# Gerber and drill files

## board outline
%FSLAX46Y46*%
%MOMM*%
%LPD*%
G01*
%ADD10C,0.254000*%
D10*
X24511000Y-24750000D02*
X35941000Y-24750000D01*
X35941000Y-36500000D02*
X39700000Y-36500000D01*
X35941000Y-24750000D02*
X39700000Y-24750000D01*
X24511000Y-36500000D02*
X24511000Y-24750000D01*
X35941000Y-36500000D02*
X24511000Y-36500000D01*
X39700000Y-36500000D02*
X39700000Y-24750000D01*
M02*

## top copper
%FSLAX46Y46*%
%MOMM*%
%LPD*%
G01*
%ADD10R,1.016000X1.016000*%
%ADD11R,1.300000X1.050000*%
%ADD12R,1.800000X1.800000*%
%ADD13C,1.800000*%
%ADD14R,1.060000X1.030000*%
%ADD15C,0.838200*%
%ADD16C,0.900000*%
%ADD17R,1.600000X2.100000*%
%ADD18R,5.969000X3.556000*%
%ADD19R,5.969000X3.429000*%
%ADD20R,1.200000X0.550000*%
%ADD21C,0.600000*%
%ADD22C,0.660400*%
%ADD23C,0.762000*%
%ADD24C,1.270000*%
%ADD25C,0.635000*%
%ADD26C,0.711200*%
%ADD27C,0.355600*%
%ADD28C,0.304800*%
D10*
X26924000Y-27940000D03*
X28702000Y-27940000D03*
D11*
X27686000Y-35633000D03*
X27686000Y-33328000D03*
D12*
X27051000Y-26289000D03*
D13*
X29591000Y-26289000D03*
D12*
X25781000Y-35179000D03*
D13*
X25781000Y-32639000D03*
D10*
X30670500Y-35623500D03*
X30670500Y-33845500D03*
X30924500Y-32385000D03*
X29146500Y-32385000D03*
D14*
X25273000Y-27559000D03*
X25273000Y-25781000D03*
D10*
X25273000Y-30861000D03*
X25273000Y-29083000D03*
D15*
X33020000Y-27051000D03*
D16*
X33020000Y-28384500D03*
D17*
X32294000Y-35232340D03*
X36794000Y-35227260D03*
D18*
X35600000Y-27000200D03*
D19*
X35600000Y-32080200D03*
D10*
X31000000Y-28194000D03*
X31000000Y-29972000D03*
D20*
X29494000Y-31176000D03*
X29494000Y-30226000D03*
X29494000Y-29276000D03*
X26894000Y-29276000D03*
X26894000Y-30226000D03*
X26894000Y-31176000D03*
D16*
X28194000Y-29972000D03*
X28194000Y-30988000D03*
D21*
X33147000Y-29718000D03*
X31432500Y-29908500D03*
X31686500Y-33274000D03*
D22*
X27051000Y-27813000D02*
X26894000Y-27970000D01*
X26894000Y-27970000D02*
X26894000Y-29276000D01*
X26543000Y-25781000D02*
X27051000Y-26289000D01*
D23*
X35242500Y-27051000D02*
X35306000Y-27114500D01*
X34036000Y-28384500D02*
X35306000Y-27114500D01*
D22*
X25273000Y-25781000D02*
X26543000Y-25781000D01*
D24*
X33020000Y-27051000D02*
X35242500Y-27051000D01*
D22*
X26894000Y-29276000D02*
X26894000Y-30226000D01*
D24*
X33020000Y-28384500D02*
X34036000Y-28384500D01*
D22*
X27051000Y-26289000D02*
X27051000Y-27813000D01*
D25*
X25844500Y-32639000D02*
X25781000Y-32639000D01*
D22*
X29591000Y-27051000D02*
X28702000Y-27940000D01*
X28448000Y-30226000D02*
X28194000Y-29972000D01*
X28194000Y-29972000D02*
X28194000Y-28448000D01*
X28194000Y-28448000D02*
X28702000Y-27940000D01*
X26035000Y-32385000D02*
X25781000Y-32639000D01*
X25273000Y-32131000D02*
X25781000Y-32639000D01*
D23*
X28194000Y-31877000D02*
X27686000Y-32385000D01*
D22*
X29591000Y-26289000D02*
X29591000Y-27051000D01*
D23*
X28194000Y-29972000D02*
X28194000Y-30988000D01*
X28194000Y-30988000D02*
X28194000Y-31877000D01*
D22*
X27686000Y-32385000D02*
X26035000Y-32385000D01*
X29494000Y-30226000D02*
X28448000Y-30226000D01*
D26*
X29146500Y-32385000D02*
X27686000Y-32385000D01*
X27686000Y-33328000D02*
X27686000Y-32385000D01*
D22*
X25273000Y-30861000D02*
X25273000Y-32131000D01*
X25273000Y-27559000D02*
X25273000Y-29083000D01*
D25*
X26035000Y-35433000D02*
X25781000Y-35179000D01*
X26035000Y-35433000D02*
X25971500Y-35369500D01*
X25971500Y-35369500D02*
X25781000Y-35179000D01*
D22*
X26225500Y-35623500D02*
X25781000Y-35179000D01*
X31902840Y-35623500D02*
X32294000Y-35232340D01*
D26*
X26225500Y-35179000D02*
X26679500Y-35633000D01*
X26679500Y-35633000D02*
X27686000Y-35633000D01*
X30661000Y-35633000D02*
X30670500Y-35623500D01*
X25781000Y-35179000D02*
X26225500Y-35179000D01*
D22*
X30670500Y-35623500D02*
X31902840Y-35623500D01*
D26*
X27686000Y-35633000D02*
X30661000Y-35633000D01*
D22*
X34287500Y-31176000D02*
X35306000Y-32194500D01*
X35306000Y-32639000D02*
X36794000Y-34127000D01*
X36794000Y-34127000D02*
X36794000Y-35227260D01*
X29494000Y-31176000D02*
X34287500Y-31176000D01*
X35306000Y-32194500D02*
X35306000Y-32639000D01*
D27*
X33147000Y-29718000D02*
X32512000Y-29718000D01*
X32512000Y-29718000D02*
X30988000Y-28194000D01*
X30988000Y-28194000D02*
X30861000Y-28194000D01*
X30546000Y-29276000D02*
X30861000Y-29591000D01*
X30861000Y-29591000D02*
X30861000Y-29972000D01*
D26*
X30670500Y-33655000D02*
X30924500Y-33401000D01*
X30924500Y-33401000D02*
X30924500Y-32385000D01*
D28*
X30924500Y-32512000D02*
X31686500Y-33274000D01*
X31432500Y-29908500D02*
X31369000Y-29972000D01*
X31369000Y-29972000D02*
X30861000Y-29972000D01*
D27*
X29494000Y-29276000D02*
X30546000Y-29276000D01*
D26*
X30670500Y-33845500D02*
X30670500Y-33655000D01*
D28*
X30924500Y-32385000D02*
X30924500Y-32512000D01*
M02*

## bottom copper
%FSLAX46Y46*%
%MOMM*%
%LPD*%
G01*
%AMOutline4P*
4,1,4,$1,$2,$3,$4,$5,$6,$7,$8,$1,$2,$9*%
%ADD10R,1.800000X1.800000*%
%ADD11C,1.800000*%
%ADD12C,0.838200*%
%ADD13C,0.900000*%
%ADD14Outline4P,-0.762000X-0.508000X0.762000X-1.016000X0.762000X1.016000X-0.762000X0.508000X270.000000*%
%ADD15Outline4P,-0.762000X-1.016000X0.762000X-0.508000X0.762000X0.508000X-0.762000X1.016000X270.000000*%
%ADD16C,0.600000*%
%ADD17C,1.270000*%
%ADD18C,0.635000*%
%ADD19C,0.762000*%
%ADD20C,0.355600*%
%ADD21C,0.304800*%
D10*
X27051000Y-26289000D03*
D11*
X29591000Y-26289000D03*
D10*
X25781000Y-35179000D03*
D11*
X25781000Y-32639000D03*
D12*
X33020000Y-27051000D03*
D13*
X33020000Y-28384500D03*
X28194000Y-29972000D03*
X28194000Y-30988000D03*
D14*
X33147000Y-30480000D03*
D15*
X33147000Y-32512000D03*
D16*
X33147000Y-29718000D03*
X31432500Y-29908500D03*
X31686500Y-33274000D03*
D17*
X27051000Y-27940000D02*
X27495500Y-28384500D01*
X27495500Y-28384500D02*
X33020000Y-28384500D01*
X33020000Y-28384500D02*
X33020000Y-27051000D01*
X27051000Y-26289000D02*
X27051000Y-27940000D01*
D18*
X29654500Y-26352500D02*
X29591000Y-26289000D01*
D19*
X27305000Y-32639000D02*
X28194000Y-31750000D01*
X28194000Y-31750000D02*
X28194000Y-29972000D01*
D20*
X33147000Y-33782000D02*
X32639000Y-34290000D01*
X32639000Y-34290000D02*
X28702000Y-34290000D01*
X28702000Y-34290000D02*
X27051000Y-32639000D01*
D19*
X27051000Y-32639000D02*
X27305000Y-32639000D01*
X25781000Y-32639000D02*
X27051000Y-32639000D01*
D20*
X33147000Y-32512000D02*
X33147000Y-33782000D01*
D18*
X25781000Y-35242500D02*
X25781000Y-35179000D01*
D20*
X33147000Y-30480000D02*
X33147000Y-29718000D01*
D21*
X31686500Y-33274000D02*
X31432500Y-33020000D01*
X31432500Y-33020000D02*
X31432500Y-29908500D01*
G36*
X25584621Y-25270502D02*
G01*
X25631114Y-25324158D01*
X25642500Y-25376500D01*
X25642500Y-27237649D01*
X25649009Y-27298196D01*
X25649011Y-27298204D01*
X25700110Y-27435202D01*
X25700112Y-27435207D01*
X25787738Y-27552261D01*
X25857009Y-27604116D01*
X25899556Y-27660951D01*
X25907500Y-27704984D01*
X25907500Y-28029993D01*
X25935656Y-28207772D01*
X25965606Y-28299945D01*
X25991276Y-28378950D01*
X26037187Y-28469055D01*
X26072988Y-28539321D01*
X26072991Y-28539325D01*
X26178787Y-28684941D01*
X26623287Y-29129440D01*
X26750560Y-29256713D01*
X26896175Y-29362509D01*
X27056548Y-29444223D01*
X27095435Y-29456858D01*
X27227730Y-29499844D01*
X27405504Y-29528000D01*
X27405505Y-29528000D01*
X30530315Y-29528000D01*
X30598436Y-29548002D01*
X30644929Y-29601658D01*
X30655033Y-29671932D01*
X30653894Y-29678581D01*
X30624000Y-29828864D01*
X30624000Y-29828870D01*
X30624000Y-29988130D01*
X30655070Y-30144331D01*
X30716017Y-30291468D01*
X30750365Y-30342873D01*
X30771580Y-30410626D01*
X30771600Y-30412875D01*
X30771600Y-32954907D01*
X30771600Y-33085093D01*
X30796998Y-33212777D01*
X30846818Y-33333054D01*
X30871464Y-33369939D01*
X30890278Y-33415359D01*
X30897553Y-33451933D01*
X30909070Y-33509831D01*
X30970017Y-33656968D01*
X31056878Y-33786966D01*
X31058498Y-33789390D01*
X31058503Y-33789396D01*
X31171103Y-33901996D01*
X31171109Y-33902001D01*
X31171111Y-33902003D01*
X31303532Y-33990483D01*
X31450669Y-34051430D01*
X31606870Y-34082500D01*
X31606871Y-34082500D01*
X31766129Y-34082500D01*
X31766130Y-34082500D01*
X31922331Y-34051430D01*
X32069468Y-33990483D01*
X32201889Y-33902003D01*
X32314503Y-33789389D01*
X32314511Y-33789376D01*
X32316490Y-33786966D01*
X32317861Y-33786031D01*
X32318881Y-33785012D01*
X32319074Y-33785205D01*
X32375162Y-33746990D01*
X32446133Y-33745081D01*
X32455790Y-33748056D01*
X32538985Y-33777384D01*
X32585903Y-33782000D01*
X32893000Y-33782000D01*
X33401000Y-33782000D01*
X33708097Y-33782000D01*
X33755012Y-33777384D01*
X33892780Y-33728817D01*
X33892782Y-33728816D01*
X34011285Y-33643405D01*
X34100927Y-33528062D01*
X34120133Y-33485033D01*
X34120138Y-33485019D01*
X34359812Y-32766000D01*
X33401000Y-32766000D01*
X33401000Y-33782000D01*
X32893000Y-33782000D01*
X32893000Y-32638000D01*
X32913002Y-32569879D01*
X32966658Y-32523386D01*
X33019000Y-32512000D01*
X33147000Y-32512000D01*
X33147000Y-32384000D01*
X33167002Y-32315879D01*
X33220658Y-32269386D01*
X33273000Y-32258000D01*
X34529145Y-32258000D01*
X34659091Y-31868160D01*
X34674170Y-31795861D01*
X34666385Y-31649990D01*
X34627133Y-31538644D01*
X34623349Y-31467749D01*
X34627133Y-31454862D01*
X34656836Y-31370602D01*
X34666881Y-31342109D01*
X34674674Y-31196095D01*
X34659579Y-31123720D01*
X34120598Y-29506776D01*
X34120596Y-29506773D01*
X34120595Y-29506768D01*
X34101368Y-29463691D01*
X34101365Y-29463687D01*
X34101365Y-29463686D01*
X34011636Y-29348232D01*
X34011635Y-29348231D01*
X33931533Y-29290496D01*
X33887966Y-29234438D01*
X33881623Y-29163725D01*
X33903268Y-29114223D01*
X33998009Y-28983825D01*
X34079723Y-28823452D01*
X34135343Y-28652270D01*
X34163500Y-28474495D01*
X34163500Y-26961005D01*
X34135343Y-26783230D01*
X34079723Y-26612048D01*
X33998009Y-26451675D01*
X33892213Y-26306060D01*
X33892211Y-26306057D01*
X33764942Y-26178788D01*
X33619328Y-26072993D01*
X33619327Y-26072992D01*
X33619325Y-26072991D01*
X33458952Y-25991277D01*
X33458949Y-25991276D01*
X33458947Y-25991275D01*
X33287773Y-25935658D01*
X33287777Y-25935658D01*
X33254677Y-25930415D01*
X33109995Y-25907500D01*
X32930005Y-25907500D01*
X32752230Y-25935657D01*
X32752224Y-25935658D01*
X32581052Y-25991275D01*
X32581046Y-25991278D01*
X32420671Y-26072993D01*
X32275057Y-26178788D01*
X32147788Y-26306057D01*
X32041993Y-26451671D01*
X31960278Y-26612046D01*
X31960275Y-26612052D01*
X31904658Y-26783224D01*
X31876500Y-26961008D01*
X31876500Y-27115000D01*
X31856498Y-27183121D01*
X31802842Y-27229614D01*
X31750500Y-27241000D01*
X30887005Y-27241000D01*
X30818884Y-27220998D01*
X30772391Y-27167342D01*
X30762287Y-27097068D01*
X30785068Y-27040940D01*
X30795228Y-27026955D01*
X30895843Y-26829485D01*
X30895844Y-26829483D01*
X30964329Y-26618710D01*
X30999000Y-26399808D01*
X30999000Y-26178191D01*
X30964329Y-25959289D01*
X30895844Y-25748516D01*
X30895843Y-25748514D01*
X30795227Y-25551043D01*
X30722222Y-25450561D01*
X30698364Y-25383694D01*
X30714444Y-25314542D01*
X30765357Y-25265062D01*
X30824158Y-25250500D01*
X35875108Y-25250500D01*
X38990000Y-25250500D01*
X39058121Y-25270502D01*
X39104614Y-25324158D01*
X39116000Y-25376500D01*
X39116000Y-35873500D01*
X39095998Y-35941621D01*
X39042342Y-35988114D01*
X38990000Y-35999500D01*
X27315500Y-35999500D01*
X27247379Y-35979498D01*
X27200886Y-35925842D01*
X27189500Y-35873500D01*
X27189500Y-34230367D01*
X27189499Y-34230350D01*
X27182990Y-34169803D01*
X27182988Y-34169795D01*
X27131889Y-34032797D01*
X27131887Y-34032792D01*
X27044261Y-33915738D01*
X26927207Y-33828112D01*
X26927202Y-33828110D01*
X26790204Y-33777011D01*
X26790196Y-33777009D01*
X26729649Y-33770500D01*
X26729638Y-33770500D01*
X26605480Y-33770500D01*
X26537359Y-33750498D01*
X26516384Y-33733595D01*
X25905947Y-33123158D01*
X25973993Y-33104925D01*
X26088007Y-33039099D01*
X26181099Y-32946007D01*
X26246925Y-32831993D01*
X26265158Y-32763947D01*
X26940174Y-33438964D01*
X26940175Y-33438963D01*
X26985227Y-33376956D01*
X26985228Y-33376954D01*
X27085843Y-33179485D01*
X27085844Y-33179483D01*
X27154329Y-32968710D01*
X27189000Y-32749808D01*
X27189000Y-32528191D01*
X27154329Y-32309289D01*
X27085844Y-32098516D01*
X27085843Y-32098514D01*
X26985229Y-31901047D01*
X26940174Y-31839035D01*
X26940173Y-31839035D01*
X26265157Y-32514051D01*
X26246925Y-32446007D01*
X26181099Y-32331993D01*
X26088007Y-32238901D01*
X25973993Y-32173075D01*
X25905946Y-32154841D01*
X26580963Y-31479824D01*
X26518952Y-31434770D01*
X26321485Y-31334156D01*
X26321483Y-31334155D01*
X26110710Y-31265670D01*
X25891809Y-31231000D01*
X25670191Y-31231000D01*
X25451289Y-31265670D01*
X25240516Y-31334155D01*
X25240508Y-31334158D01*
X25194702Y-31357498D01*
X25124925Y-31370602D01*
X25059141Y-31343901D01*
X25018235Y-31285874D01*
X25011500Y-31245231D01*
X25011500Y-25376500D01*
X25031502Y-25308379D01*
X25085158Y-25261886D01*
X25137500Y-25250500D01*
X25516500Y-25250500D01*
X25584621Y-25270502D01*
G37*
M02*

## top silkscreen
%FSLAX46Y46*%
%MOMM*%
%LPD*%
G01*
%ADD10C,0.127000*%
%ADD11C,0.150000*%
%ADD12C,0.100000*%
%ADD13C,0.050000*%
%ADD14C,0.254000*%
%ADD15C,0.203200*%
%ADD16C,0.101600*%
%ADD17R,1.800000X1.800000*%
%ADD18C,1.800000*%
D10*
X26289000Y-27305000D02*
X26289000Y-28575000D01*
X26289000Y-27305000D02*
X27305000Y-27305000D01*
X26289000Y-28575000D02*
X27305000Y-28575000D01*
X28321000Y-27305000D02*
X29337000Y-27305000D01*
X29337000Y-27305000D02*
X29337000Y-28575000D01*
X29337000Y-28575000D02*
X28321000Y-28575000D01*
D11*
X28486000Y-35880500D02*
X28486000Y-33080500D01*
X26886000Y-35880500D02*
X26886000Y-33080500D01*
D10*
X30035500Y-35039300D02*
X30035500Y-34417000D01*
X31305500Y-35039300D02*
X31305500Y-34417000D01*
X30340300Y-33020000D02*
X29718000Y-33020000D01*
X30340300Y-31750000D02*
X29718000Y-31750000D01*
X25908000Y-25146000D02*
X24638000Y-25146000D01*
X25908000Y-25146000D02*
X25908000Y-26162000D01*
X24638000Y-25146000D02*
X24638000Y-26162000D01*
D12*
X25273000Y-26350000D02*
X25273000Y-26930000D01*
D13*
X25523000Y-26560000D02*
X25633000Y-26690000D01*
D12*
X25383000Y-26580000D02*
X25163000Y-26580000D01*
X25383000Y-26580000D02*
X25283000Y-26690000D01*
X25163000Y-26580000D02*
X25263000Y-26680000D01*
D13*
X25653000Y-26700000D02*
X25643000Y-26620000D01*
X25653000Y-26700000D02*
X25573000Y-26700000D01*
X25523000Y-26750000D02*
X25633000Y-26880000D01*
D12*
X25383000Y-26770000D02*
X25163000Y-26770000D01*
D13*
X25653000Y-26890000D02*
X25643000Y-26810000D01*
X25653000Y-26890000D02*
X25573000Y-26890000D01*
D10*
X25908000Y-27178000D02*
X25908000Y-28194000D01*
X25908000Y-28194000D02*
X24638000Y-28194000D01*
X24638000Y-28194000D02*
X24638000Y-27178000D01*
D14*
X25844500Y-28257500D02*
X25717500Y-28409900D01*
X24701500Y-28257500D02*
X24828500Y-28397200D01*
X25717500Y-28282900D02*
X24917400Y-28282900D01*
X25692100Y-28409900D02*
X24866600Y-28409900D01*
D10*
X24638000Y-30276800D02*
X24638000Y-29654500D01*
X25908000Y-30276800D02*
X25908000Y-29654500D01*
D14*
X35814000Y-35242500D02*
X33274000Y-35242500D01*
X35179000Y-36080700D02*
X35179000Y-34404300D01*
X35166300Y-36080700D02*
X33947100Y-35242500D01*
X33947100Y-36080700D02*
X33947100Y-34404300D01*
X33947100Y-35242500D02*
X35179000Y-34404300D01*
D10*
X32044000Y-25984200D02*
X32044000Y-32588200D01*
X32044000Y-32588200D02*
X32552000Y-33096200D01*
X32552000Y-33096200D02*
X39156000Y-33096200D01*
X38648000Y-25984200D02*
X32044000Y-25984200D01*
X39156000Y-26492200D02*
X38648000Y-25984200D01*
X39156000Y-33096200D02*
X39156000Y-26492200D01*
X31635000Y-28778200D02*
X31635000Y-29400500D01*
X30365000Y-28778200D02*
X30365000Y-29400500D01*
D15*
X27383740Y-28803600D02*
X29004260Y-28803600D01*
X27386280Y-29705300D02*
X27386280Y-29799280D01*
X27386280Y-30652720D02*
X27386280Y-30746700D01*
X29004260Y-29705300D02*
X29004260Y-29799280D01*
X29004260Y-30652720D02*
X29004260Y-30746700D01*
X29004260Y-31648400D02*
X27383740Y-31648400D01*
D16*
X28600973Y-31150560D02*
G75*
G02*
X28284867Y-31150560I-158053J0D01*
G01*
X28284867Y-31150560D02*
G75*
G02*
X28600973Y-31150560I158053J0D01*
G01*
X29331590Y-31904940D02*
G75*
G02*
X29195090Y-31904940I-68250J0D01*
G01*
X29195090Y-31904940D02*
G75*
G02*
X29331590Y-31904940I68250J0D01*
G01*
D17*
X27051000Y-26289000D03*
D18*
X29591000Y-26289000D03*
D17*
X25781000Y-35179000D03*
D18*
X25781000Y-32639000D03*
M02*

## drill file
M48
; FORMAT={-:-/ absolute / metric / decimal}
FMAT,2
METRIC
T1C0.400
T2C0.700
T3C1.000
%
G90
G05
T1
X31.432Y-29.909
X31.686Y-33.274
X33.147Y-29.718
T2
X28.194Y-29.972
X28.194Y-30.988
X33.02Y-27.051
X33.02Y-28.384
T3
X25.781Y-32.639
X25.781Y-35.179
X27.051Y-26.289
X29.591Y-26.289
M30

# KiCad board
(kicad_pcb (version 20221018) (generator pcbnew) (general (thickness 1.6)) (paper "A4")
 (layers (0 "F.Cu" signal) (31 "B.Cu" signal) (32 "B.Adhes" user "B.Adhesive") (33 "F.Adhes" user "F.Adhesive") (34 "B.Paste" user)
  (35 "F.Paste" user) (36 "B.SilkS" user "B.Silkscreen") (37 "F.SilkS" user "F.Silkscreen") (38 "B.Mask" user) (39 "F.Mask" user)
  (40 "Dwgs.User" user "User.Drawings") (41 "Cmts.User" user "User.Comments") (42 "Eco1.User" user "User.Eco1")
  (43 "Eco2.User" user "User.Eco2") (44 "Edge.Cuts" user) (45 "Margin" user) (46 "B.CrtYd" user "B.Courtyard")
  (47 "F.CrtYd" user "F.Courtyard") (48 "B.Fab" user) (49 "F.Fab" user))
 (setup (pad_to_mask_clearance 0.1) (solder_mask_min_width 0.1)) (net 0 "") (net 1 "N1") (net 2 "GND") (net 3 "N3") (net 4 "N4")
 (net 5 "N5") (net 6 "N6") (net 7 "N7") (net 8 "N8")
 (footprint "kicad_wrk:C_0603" (layer "F.Cu") (at 27.813 27.94)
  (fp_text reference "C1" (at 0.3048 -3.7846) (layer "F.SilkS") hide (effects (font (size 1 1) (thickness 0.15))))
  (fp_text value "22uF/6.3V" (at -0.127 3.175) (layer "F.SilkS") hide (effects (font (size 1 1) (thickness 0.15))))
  (fp_line (start -1.524 -0.635) (end -1.524 0.635) (stroke (width 0.127) (type solid)) (layer "F.SilkS"))
  (fp_line (start -1.524 -0.635) (end -0.508 -0.635) (stroke (width 0.127) (type solid)) (layer "F.SilkS"))
  (fp_line (start -1.524 0.635) (end -0.508 0.635) (stroke (width 0.127) (type solid)) (layer "F.SilkS"))
  (fp_line (start 0.508 -0.635) (end 1.524 -0.635) (stroke (width 0.127) (type solid)) (layer "F.SilkS"))
  (fp_line (start 1.524 -0.635) (end 1.524 0.635) (stroke (width 0.127) (type solid)) (layer "F.SilkS"))
  (fp_line (start 1.524 0.635) (end 0.508 0.635) (stroke (width 0.127) (type solid)) (layer "F.SilkS"))
  (pad "1" smd rect (at -0.889 0) (size 1.016 1.016) (layers "F.Cu" "F.Paste" "F.Mask") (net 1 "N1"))
  (pad "2" smd rect (at 0.889 0) (size 1.016 1.016) (layers "F.Cu" "F.Paste" "F.Mask") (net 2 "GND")))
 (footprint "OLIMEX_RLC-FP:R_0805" (layer "F.Cu") (at 27.686 34.4805 180)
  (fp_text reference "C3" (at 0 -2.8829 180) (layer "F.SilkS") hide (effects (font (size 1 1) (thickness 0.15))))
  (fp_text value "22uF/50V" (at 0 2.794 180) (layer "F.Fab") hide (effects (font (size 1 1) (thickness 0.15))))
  (fp_line (start -0.8 -1.4) (end -0.8 1.4) (stroke (width 0.15) (type solid)) (layer "F.SilkS"))
  (fp_line (start 0.8 -1.4) (end 0.8 1.4) (stroke (width 0.15) (type solid)) (layer "F.SilkS"))
  (pad "1" smd rect (at 0 -1.1525 180) (size 1.3 1.05) (layers "F.Cu" "F.Paste" "F.Mask") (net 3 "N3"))
  (pad "2" smd rect (at 0 1.1525 180) (size 1.3 1.05) (layers "F.Cu" "F.Paste" "F.Mask") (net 2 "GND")))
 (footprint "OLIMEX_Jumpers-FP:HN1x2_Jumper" (layer "F.Cu") (at 28.321 26.289)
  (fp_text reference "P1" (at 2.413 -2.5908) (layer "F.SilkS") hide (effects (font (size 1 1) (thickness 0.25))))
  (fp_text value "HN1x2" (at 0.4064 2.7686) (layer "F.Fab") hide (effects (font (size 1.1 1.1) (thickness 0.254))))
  (pad "1" thru_hole rect (at -1.27 0 90) (size 1.8 1.8) (drill 1) (layers "*.Cu" "*.Mask" "F.SilkS") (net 1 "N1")
   (solder_mask_margin 0.0508) (solder_paste_margin -0.0508))
  (pad "2" thru_hole circle (at 1.27 0 90) (size 1.8 1.8) (drill 1) (layers "*.Cu" "*.Mask" "F.SilkS") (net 2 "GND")
   (solder_mask_margin 0.0508) (solder_paste_margin -0.0508)))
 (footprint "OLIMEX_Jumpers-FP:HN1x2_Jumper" (layer "F.Cu") (at 25.781 33.909 90)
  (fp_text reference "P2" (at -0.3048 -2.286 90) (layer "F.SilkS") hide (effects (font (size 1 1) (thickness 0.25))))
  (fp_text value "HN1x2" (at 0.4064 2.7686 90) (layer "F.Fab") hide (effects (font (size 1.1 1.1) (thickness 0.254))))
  (pad "1" thru_hole rect (at -1.27 0 180) (size 1.8 1.8) (drill 1) (layers "*.Cu" "*.Mask" "F.SilkS") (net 3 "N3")
   (solder_mask_margin 0.0508) (solder_paste_margin -0.0508))
  (pad "2" thru_hole circle (at 1.27 0 180) (size 1.8 1.8) (drill 1) (layers "*.Cu" "*.Mask" "F.SilkS") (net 2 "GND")
   (solder_mask_margin 0.0508) (solder_paste_margin -0.0508)))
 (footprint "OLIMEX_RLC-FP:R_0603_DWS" (layer "F.Cu") (at 30.6705 34.7345 90)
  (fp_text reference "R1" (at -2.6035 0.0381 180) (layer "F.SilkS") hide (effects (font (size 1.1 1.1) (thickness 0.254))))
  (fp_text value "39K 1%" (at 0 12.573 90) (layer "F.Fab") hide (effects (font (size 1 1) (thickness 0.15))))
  (fp_line (start -0.3048 -0.635) (end 0.3175 -0.635) (stroke (width 0.127) (type solid)) (layer "F.SilkS"))
  (fp_line (start -0.3048 0.635) (end 0.3175 0.635) (stroke (width 0.127) (type solid)) (layer "F.SilkS"))
  (pad "1" smd rect (at -0.889 0 90) (size 1.016 1.016) (layers "F.Cu" "F.Paste" "F.Mask") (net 3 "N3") (solder_mask_margin 0.0508)
   (solder_paste_margin -0.0508) (clearance 0.0508))
  (pad "2" smd rect (at 0.889 0 90) (size 1.016 1.016) (layers "F.Cu" "F.Paste" "F.Mask") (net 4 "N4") (solder_mask_margin 0.0508)
   (solder_paste_margin -0.0508) (clearance 0.0508)))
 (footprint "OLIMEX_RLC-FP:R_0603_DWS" (layer "F.Cu") (at 30.0355 32.385 180)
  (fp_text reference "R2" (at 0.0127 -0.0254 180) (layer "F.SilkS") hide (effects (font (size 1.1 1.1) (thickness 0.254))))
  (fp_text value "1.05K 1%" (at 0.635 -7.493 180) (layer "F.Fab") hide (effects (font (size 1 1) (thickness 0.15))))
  (fp_line (start -0.3048 -0.635) (end 0.3175 -0.635) (stroke (width 0.127) (type solid)) (layer "F.SilkS"))
  (fp_line (start -0.3048 0.635) (end 0.3175 0.635) (stroke (width 0.127) (type solid)) (layer "F.SilkS"))
  (pad "1" smd rect (at -0.889 0 180) (size 1.016 1.016) (layers "F.Cu" "F.Paste" "F.Mask") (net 4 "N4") (solder_mask_margin 0.0508)
   (solder_paste_margin -0.0508) (clearance 0.0508))
  (pad "2" smd rect (at 0.889 0 180) (size 1.016 1.016) (layers "F.Cu" "F.Paste" "F.Mask") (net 2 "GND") (solder_mask_margin 0.0508)
   (solder_paste_margin -0.0508) (clearance 0.0508)))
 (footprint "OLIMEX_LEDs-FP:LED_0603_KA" (layer "F.Cu") (at 25.273 26.67 -90)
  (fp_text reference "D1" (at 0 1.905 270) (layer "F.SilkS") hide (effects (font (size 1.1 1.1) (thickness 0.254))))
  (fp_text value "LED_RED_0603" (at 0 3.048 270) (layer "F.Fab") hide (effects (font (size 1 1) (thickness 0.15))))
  (fp_line (start -1.524 -0.635) (end -1.524 0.635) (stroke (width 0.127) (type solid)) (layer "F.SilkS"))
  (fp_line (start -1.524 -0.635) (end -0.508 -0.635) (stroke (width 0.127) (type solid)) (layer "F.SilkS"))
  (fp_line (start -1.524 0.635) (end -0.508 0.635) (stroke (width 0.127) (type solid)) (layer "F.SilkS"))
  (fp_line (start -0.32 0) (end 0.26 0) (stroke (width 0.1) (type solid)) (layer "F.SilkS"))
  (fp_line (start -0.11 -0.25) (end 0.02 -0.36) (stroke (width 0.05) (type solid)) (layer "F.SilkS"))
  (fp_line (start -0.09 -0.11) (end -0.09 0.11) (stroke (width 0.1) (type solid)) (layer "F.SilkS"))
  (fp_line (start -0.09 -0.11) (end 0.02 -0.01) (stroke (width 0.1) (type solid)) (layer "F.SilkS"))
  (fp_line (start -0.09 0.11) (end 0.01 0.01) (stroke (width 0.1) (type solid)) (layer "F.SilkS"))
  (fp_line (start 0.03 -0.38) (end -0.05 -0.37) (stroke (width 0.05) (type solid)) (layer "F.SilkS"))
  (fp_line (start 0.03 -0.38) (end 0.03 -0.3) (stroke (width 0.05) (type solid)) (layer "F.SilkS"))
  (fp_line (start 0.08 -0.25) (end 0.21 -0.36) (stroke (width 0.05) (type solid)) (layer "F.SilkS"))
  (fp_line (start 0.1 -0.11) (end 0.1 0.11) (stroke (width 0.1) (type solid)) (layer "F.SilkS"))
  (fp_line (start 0.22 -0.38) (end 0.14 -0.37) (stroke (width 0.05) (type solid)) (layer "F.SilkS"))
  (fp_line (start 0.22 -0.38) (end 0.22 -0.3) (stroke (width 0.05) (type solid)) (layer "F.SilkS"))
  (fp_line (start 0.508 -0.635) (end 1.524 -0.635) (stroke (width 0.127) (type solid)) (layer "F.SilkS"))
  (fp_line (start 1.524 -0.635) (end 1.524 0.635) (stroke (width 0.127) (type solid)) (layer "F.SilkS"))
  (fp_line (start 1.524 0.635) (end 0.508 0.635) (stroke (width 0.127) (type solid)) (layer "F.SilkS"))
  (fp_line (start 1.5875 -0.5715) (end 1.7399 -0.4445) (stroke (width 0.254) (type solid)) (layer "F.SilkS"))
  (fp_line (start 1.5875 0.5715) (end 1.7272 0.4445) (stroke (width 0.254) (type solid)) (layer "F.SilkS"))
  (fp_line (start 1.6129 -0.4445) (end 1.6129 0.3556) (stroke (width 0.254) (type solid)) (layer "F.SilkS"))
  (fp_line (start 1.7399 -0.4191) (end 1.7399 0.4064) (stroke (width 0.254) (type solid)) (layer "F.SilkS"))
  (pad "1" smd rect (at 0.889 0 270) (size 1.03 1.06) (layers "F.Cu" "F.Paste" "F.Mask") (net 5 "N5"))
  (pad "2" smd rect (at -0.889 0 270) (size 1.03 1.06) (layers "F.Cu" "F.Paste" "F.Mask") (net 1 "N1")))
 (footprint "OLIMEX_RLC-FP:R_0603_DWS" (layer "F.Cu") (at 25.273 29.972 90)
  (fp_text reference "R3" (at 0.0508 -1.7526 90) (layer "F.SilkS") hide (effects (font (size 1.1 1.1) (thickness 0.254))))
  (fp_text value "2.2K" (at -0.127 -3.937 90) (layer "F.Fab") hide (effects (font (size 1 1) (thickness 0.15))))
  (fp_line (start -0.3048 -0.635) (end 0.3175 -0.635) (stroke (width 0.127) (type solid)) (layer "F.SilkS"))
  (fp_line (start -0.3048 0.635) (end 0.3175 0.635) (stroke (width 0.127) (type solid)) (layer "F.SilkS"))
  (pad "1" smd rect (at -0.889 0 90) (size 1.016 1.016) (layers "F.Cu" "F.Paste" "F.Mask") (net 2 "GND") (solder_mask_margin 0.0508)
   (solder_paste_margin -0.0508) (clearance 0.0508))
  (pad "2" smd rect (at 0.889 0 90) (size 1.016 1.016) (layers "F.Cu" "F.Paste" "F.Mask") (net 5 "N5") (solder_mask_margin 0.0508)
   (solder_paste_margin -0.0508) (clearance 0.0508)))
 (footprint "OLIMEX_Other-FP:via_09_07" (layer "F.Cu") (at 33.02 27.051 180)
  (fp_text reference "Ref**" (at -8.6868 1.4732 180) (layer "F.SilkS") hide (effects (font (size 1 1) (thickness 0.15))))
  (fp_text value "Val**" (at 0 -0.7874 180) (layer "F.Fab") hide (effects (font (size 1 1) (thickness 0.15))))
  (pad "0" thru_hole circle (at 0 0 180) (size 0.8382 0.8382) (drill 0.7) (layers "*.Cu") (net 1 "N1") (zone_connect 2)))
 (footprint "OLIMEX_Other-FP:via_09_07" (layer "F.Cu") (at 33.02 28.321 180)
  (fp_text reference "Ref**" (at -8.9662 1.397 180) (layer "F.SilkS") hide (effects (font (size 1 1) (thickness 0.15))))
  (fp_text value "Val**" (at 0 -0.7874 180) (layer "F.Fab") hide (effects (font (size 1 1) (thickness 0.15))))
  (pad "0" thru_hole circle (at 0 -0.0635 180) (size 0.9 0.9) (drill 0.7) (layers "*.Cu") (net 1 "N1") (zone_connect 2)))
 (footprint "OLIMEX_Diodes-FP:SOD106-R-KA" (layer "F.Cu") (at 34.544 35.2425 180)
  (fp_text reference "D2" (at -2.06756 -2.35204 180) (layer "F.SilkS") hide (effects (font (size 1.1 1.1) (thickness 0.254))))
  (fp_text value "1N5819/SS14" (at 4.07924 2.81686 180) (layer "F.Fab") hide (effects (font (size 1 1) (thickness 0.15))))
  (fp_line (start -1.27 0) (end 1.27 0) (stroke (width 0.254) (type solid)) (layer "F.SilkS"))
  (fp_line (start -0.635 -0.8382) (end -0.635 0.8382) (stroke (width 0.254) (type solid)) (layer "F.SilkS"))
  (fp_line (start -0.6223 -0.8382) (end 0.5969 0) (stroke (width 0.254) (type solid)) (layer "F.SilkS"))
  (fp_line (start 0.5969 -0.8382) (end 0.5969 0.8382) (stroke (width 0.254) (type solid)) (layer "F.SilkS"))
  (fp_line (start 0.5969 0) (end -0.635 0.8382) (stroke (width 0.254) (type solid)) (layer "F.SilkS"))
  (pad "1" smd rect (at 2.25 0.01016 180) (size 1.6 2.1) (layers "F.Cu" "F.Paste" "F.Mask") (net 3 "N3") (solder_mask_margin 0.0508)
   (solder_paste_margin -0.0508) (clearance 0.0508))
  (pad "2" smd rect (at -2.25 0.01524 180) (size 1.6 2.1) (layers "F.Cu" "F.Paste" "F.Mask") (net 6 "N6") (solder_mask_margin 0.0508)
   (solder_paste_margin -0.0508) (clearance 0.0508)))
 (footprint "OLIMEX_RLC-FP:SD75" (layer "F.Cu") (at 35.6 29.5402)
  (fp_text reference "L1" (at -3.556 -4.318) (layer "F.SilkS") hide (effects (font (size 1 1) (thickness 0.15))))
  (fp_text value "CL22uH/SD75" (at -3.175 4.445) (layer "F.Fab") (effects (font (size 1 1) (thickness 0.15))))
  (fp_line (start -3.556 -3.556) (end -3.556 3.048) (stroke (width 0.127) (type solid)) (layer "F.SilkS"))
  (fp_line (start -3.556 3.048) (end -3.048 3.556) (stroke (width 0.127) (type solid)) (layer "F.SilkS"))
  (fp_line (start -3.048 3.556) (end 3.556 3.556) (stroke (width 0.127) (type solid)) (layer "F.SilkS"))
  (fp_line (start 3.048 -3.556) (end -3.556 -3.556) (stroke (width 0.127) (type solid)) (layer "F.SilkS"))
  (fp_line (start 3.556 -3.048) (end 3.048 -3.556) (stroke (width 0.127) (type solid)) (layer "F.SilkS"))
  (fp_line (start 3.556 3.556) (end 3.556 -3.048) (stroke (width 0.127) (type solid)) (layer "F.SilkS"))
  (pad "1" smd rect (at 0 -2.54) (size 5.969 3.556) (layers "F.Cu" "F.Paste" "F.Mask") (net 1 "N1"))
  (pad "2" smd rect (at 0 2.54) (size 5.969 3.429) (layers "F.Cu" "F.Paste" "F.Mask") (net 6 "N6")))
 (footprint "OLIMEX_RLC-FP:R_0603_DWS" (layer "F.Cu") (at 31 29.083 -90)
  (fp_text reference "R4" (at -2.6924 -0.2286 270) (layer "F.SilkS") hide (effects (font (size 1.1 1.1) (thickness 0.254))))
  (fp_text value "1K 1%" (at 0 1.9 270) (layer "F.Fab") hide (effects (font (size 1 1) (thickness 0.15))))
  (fp_line (start -0.3048 -0.635) (end 0.3175 -0.635) (stroke (width 0.127) (type solid)) (layer "F.SilkS"))
  (fp_line (start -0.3048 0.635) (end 0.3175 0.635) (stroke (width 0.127) (type solid)) (layer "F.SilkS"))
  (pad "1" smd rect (at -0.889 0 270) (size 1.016 1.016) (layers "F.Cu" "F.Paste" "F.Mask") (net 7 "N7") (solder_mask_margin 0.0508)
   (solder_paste_margin -0.0508) (clearance 0.0508))
  (pad "2" smd rect (at 0.889 0 270) (size 1.016 1.016) (layers "F.Cu" "F.Paste" "F.Mask") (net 4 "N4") (solder_mask_margin 0.0508)
   (solder_paste_margin -0.0508) (clearance 0.0508)))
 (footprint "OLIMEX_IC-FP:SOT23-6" (layer "F.Cu") (at 28.194 30.226)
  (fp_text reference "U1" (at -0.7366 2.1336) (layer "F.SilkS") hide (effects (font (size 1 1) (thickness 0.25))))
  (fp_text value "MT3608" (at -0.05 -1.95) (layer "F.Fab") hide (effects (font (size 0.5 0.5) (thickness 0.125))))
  (fp_line (start -0.81026 -1.4224) (end 0.81026 -1.4224) (stroke (width 0.2032) (type solid)) (layer "F.SilkS"))
  (fp_line (start -0.80772 -0.5207) (end -0.80772 -0.42672) (stroke (width 0.2032) (type solid)) (layer "F.SilkS"))
  (fp_line (start -0.80772 0.42672) (end -0.80772 0.5207) (stroke (width 0.2032) (type solid)) (layer "F.SilkS"))
  (fp_line (start 0.81026 -0.5207) (end 0.81026 -0.42672) (stroke (width 0.2032) (type solid)) (layer "F.SilkS"))
  (fp_line (start 0.81026 0.42672) (end 0.81026 0.5207) (stroke (width 0.2032) (type solid)) (layer "F.SilkS"))
  (fp_line (start 0.81026 1.4224) (end -0.81026 1.4224) (stroke (width 0.2032) (type solid)) (layer "F.SilkS"))
  (fp_circle (center 0.24892 0.92456) (end 0.36068 1.03632) (stroke (width 0.1016) (type solid)) (fill none) (layer "F.SilkS"))
  (fp_circle (center 1.06934 1.67894) (end 1.1176 1.7272) (stroke (width 0.1016) (type solid)) (fill none) (layer "F.SilkS"))
  (pad "1" smd rect (at 1.3 0.95 90) (size 0.55 1.2) (layers "F.Cu" "F.Paste" "F.Mask") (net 6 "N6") (solder_mask_margin 0.0508)
   (solder_paste_margin -0.0508) (clearance 0.0508))
  (pad "2" smd rect (at 1.3 0 90) (size 0.55 1.2) (layers "F.Cu" "F.Paste" "F.Mask") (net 2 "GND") (solder_mask_margin 0.0508)
   (solder_paste_margin -0.0508) (clearance 0.0508))
  (pad "3" smd rect (at 1.3 -0.95 90) (size 0.55 1.2) (layers "F.Cu" "F.Paste" "F.Mask") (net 4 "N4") (solder_mask_margin 0.0508)
   (solder_paste_margin -0.0508) (clearance 0.0508))
  (pad "4" smd rect (at -1.3 -0.95 90) (size 0.55 1.2) (layers "F.Cu" "F.Paste" "F.Mask") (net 1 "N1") (solder_mask_margin 0.0508)
   (solder_paste_margin -0.0508) (clearance 0.0508))
  (pad "5" smd rect (at -1.3 0 90) (size 0.55 1.2) (layers "F.Cu" "F.Paste" "F.Mask") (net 1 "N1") (solder_mask_margin 0.0508)
   (solder_paste_margin -0.0508) (clearance 0.0508))
  (pad "6" smd rect (at -1.3 0.95 90) (size 0.55 1.2) (layers "F.Cu" "F.Paste" "F.Mask") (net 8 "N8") (solder_mask_margin 0.0508)
   (solder_paste_margin -0.0508) (clearance 0.0508)))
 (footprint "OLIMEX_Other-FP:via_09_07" (layer "F.Cu") (at 28.194 29.972)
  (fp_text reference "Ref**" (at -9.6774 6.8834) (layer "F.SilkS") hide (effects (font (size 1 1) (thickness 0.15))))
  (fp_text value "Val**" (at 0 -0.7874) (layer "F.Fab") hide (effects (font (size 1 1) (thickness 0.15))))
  (pad "0" thru_hole circle (at 0 0) (size 0.9 0.9) (drill 0.7) (layers "*.Cu") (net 2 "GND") (zone_connect 2)))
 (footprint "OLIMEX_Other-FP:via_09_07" (layer "F.Cu") (at 28.194 30.988)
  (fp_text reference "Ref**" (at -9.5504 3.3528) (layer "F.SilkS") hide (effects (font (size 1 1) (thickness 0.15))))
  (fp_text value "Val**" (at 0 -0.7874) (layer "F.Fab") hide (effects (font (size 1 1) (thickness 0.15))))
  (pad "0" thru_hole circle (at 0 0) (size 0.9 0.9) (drill 0.7) (layers "*.Cu") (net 2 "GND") (zone_connect 2)))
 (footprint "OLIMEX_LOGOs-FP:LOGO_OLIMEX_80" (layer "B.Cu") (at 35.8775 27.686 180)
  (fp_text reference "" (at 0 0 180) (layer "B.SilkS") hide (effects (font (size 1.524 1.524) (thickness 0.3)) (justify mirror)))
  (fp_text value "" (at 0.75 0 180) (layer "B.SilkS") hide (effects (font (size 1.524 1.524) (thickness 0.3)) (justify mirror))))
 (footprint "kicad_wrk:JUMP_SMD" (layer "B.Cu") (at 33.147 31.496 -90)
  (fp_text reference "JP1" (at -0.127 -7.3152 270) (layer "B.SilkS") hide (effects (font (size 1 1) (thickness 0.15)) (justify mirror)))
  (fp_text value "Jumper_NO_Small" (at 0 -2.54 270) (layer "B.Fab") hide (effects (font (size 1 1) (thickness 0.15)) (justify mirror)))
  (pad "1" smd trapezoid (at -1.016 0 270) (size 1.524 1.524) (rect_delta -0.508 0) (layers "B.Cu" "B.Mask") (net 7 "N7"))
  (pad "2" smd trapezoid (at 1.016 0 270) (size 1.524 1.524) (rect_delta 0.508 0) (layers "B.Cu" "B.Mask") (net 2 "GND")))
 (gr_line (start 24.511 24.75) (end 35.941 24.75) (stroke (width 0.254) (type solid)) (layer "Edge.Cuts"))
 (gr_line (start 35.941 36.5) (end 39.7 36.5) (stroke (width 0.254) (type solid)) (layer "Edge.Cuts"))
 (gr_line (start 35.941 24.75) (end 39.7 24.75) (stroke (width 0.254) (type solid)) (layer "Edge.Cuts"))
 (gr_line (start 24.511 36.5) (end 24.511 24.75) (stroke (width 0.254) (type solid)) (layer "Edge.Cuts"))
 (gr_line (start 35.941 36.5) (end 24.511 36.5) (stroke (width 0.254) (type solid)) (layer "Edge.Cuts"))
 (gr_line (start 39.7 36.5) (end 39.7 24.75) (stroke (width 0.254) (type solid)) (layer "Edge.Cuts"))
 (segment (start 27.051 27.813) (end 26.894 27.97) (width 0.6604) (layer "F.Cu") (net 1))
 (segment (start 26.894 27.97) (end 26.894 29.276) (width 0.6604) (layer "F.Cu") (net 1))
 (segment (start 26.543 25.781) (end 27.051 26.289) (width 0.6604) (layer "F.Cu") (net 1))
 (segment (start 35.2425 27.051) (end 35.306 27.1145) (width 0.762) (layer "F.Cu") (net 1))
 (segment (start 34.036 28.3845) (end 35.306 27.1145) (width 0.762) (layer "F.Cu") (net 1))
 (segment (start 25.273 25.781) (end 26.543 25.781) (width 0.6604) (layer "F.Cu") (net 1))
 (segment (start 33.02 27.051) (end 35.2425 27.051) (width 1.27) (layer "F.Cu") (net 1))
 (segment (start 26.894 29.276) (end 26.894 30.226) (width 0.6604) (layer "F.Cu") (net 1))
 (segment (start 33.02 28.3845) (end 34.036 28.3845) (width 1.27) (layer "F.Cu") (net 1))
 (segment (start 27.051 26.289) (end 27.051 27.813) (width 0.6604) (layer "F.Cu") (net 1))
 (segment (start 27.051 27.94) (end 27.4955 28.3845) (width 1.27) (layer "B.Cu") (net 1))
 (segment (start 27.4955 28.3845) (end 33.02 28.3845) (width 1.27) (layer "B.Cu") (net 1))
 (segment (start 33.02 28.3845) (end 33.02 27.051) (width 1.27) (layer "B.Cu") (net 1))
 (segment (start 27.051 26.289) (end 27.051 27.94) (width 1.27) (layer "B.Cu") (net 1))
 (segment (start 25.8445 32.639) (end 25.781 32.639) (width 0.635) (layer "F.Cu") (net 2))
 (segment (start 29.591 27.051) (end 28.702 27.94) (width 0.6604) (layer "F.Cu") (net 2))
 (segment (start 28.448 30.226) (end 28.194 29.972) (width 0.6604) (layer "F.Cu") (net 2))
 (segment (start 28.194 29.972) (end 28.194 28.448) (width 0.6604) (layer "F.Cu") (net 2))
 (segment (start 28.194 28.448) (end 28.702 27.94) (width 0.6604) (layer "F.Cu") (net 2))
 (segment (start 26.035 32.385) (end 25.781 32.639) (width 0.6604) (layer "F.Cu") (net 2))
 (segment (start 25.273 32.131) (end 25.781 32.639) (width 0.6604) (layer "F.Cu") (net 2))
 (segment (start 28.194 31.877) (end 27.686 32.385) (width 0.762) (layer "F.Cu") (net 2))
 (segment (start 29.591 26.289) (end 29.591 27.051) (width 0.6604) (layer "F.Cu") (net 2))
 (segment (start 28.194 29.972) (end 28.194 30.988) (width 0.762) (layer "F.Cu") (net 2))
 (segment (start 28.194 30.988) (end 28.194 31.877) (width 0.762) (layer "F.Cu") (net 2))
 (segment (start 27.686 32.385) (end 26.035 32.385) (width 0.6604) (layer "F.Cu") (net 2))
 (segment (start 29.494 30.226) (end 28.448 30.226) (width 0.6604) (layer "F.Cu") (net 2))
 (segment (start 29.1465 32.385) (end 27.686 32.385) (width 0.7112) (layer "F.Cu") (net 2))
 (segment (start 27.686 33.328) (end 27.686 32.385) (width 0.7112) (layer "F.Cu") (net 2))
 (segment (start 25.273 30.861) (end 25.273 32.131) (width 0.6604) (layer "F.Cu") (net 2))
 (segment (start 29.6545 26.3525) (end 29.591 26.289) (width 0.635) (layer "B.Cu") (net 2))
 (segment (start 27.305 32.639) (end 28.194 31.75) (width 0.762) (layer "B.Cu") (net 2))
 (segment (start 28.194 31.75) (end 28.194 29.972) (width 0.762) (layer "B.Cu") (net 2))
 (segment (start 33.147 33.782) (end 32.639 34.29) (width 0.3556) (layer "B.Cu") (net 2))
 (segment (start 32.639 34.29) (end 28.702 34.29) (width 0.3556) (layer "B.Cu") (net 2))
 (segment (start 28.702 34.29) (end 27.051 32.639) (width 0.3556) (layer "B.Cu") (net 2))
 (segment (start 27.051 32.639) (end 27.305 32.639) (width 0.762) (layer "B.Cu") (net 2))
 (segment (start 25.781 32.639) (end 27.051 32.639) (width 0.762) (layer "B.Cu") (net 2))
 (segment (start 33.147 32.512) (end 33.147 33.782) (width 0.3556) (layer "B.Cu") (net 2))
 (segment (start 25.273 27.559) (end 25.273 29.083) (width 0.6604) (layer "F.Cu") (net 5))
 (segment (start 26.035 35.433) (end 25.781 35.179) (width 0.635) (layer "F.Cu") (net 3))
 (segment (start 26.035 35.433) (end 25.9715 35.3695) (width 0.635) (layer "F.Cu") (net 3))
 (segment (start 25.9715 35.3695) (end 25.781 35.179) (width 0.635) (layer "F.Cu") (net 3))
 (segment (start 26.2255 35.6235) (end 25.781 35.179) (width 0.6604) (layer "F.Cu") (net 3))
 (segment (start 31.90284 35.6235) (end 32.294 35.23234) (width 0.6604) (layer "F.Cu") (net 3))
 (segment (start 26.2255 35.179) (end 26.6795 35.633) (width 0.7112) (layer "F.Cu") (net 3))
 (segment (start 26.6795 35.633) (end 27.686 35.633) (width 0.7112) (layer "F.Cu") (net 3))
 (segment (start 30.661 35.633) (end 30.6705 35.6235) (width 0.7112) (layer "F.Cu") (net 3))
 (segment (start 25.781 35.179) (end 26.2255 35.179) (width 0.7112) (layer "F.Cu") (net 3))
 (segment (start 30.6705 35.6235) (end 31.90284 35.6235) (width 0.6604) (layer "F.Cu") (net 3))
 (segment (start 27.686 35.633) (end 30.661 35.633) (width 0.7112) (layer "F.Cu") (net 3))
 (segment (start 25.781 35.2425) (end 25.781 35.179) (width 0.635) (layer "B.Cu") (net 3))
 (segment (start 34.2875 31.176) (end 35.306 32.1945) (width 0.6604) (layer "F.Cu") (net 6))
 (segment (start 35.306 32.639) (end 36.794 34.127) (width 0.6604) (layer "F.Cu") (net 6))
 (segment (start 36.794 34.127) (end 36.794 35.22726) (width 0.6604) (layer "F.Cu") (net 6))
 (segment (start 29.494 31.176) (end 34.2875 31.176) (width 0.6604) (layer "F.Cu") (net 6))
 (segment (start 35.306 32.1945) (end 35.306 32.639) (width 0.6604) (layer "F.Cu") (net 6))
 (segment (start 33.147 29.718) (end 32.512 29.718) (width 0.3556) (layer "F.Cu") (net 7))
 (segment (start 32.512 29.718) (end 30.988 28.194) (width 0.3556) (layer "F.Cu") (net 7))
 (segment (start 30.988 28.194) (end 30.861 28.194) (width 0.3556) (layer "F.Cu") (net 7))
 (via (at 33.147 29.718) (size 0.6) (drill 0.4) (layers "F.Cu" "B.Cu") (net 7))
 (segment (start 33.147 30.48) (end 33.147 29.718) (width 0.3556) (layer "B.Cu") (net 7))
 (segment (start 30.546 29.276) (end 30.861 29.591) (width 0.3556) (layer "F.Cu") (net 4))
 (segment (start 30.861 29.591) (end 30.861 29.972) (width 0.3556) (layer "F.Cu") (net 4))
 (segment (start 30.6705 33.655) (end 30.9245 33.401) (width 0.7112) (layer "F.Cu") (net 4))
 (segment (start 30.9245 33.401) (end 30.9245 32.385) (width 0.7112) (layer "F.Cu") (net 4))
 (segment (start 30.9245 32.512) (end 31.6865 33.274) (width 0.3048) (layer "F.Cu") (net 4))
 (segment (start 31.4325 29.9085) (end 31.369 29.972) (width 0.3048) (layer "F.Cu") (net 4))
 (segment (start 31.369 29.972) (end 30.861 29.972) (width 0.3048) (layer "F.Cu") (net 4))
 (segment (start 29.494 29.276) (end 30.546 29.276) (width 0.3556) (layer "F.Cu") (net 4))
 (segment (start 30.6705 33.8455) (end 30.6705 33.655) (width 0.7112) (layer "F.Cu") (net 4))
 (segment (start 30.9245 32.385) (end 30.9245 32.512) (width 0.3048) (layer "F.Cu") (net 4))
 (via (at 31.4325 29.9085) (size 0.6) (drill 0.4) (layers "F.Cu" "B.Cu") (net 4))
 (via (at 31.6865 33.274) (size 0.6) (drill 0.4) (layers "F.Cu" "B.Cu") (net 4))
 (segment (start 31.6865 33.274) (end 31.4325 33.02) (width 0.3048) (layer "B.Cu") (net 4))
 (segment (start 31.4325 33.02) (end 31.4325 29.9085) (width 0.3048) (layer "B.Cu") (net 4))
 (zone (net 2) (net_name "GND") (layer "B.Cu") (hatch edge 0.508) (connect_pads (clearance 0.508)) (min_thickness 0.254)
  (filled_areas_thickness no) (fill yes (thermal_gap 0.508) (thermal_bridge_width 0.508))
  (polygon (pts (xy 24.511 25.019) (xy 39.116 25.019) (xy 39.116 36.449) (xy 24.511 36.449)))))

